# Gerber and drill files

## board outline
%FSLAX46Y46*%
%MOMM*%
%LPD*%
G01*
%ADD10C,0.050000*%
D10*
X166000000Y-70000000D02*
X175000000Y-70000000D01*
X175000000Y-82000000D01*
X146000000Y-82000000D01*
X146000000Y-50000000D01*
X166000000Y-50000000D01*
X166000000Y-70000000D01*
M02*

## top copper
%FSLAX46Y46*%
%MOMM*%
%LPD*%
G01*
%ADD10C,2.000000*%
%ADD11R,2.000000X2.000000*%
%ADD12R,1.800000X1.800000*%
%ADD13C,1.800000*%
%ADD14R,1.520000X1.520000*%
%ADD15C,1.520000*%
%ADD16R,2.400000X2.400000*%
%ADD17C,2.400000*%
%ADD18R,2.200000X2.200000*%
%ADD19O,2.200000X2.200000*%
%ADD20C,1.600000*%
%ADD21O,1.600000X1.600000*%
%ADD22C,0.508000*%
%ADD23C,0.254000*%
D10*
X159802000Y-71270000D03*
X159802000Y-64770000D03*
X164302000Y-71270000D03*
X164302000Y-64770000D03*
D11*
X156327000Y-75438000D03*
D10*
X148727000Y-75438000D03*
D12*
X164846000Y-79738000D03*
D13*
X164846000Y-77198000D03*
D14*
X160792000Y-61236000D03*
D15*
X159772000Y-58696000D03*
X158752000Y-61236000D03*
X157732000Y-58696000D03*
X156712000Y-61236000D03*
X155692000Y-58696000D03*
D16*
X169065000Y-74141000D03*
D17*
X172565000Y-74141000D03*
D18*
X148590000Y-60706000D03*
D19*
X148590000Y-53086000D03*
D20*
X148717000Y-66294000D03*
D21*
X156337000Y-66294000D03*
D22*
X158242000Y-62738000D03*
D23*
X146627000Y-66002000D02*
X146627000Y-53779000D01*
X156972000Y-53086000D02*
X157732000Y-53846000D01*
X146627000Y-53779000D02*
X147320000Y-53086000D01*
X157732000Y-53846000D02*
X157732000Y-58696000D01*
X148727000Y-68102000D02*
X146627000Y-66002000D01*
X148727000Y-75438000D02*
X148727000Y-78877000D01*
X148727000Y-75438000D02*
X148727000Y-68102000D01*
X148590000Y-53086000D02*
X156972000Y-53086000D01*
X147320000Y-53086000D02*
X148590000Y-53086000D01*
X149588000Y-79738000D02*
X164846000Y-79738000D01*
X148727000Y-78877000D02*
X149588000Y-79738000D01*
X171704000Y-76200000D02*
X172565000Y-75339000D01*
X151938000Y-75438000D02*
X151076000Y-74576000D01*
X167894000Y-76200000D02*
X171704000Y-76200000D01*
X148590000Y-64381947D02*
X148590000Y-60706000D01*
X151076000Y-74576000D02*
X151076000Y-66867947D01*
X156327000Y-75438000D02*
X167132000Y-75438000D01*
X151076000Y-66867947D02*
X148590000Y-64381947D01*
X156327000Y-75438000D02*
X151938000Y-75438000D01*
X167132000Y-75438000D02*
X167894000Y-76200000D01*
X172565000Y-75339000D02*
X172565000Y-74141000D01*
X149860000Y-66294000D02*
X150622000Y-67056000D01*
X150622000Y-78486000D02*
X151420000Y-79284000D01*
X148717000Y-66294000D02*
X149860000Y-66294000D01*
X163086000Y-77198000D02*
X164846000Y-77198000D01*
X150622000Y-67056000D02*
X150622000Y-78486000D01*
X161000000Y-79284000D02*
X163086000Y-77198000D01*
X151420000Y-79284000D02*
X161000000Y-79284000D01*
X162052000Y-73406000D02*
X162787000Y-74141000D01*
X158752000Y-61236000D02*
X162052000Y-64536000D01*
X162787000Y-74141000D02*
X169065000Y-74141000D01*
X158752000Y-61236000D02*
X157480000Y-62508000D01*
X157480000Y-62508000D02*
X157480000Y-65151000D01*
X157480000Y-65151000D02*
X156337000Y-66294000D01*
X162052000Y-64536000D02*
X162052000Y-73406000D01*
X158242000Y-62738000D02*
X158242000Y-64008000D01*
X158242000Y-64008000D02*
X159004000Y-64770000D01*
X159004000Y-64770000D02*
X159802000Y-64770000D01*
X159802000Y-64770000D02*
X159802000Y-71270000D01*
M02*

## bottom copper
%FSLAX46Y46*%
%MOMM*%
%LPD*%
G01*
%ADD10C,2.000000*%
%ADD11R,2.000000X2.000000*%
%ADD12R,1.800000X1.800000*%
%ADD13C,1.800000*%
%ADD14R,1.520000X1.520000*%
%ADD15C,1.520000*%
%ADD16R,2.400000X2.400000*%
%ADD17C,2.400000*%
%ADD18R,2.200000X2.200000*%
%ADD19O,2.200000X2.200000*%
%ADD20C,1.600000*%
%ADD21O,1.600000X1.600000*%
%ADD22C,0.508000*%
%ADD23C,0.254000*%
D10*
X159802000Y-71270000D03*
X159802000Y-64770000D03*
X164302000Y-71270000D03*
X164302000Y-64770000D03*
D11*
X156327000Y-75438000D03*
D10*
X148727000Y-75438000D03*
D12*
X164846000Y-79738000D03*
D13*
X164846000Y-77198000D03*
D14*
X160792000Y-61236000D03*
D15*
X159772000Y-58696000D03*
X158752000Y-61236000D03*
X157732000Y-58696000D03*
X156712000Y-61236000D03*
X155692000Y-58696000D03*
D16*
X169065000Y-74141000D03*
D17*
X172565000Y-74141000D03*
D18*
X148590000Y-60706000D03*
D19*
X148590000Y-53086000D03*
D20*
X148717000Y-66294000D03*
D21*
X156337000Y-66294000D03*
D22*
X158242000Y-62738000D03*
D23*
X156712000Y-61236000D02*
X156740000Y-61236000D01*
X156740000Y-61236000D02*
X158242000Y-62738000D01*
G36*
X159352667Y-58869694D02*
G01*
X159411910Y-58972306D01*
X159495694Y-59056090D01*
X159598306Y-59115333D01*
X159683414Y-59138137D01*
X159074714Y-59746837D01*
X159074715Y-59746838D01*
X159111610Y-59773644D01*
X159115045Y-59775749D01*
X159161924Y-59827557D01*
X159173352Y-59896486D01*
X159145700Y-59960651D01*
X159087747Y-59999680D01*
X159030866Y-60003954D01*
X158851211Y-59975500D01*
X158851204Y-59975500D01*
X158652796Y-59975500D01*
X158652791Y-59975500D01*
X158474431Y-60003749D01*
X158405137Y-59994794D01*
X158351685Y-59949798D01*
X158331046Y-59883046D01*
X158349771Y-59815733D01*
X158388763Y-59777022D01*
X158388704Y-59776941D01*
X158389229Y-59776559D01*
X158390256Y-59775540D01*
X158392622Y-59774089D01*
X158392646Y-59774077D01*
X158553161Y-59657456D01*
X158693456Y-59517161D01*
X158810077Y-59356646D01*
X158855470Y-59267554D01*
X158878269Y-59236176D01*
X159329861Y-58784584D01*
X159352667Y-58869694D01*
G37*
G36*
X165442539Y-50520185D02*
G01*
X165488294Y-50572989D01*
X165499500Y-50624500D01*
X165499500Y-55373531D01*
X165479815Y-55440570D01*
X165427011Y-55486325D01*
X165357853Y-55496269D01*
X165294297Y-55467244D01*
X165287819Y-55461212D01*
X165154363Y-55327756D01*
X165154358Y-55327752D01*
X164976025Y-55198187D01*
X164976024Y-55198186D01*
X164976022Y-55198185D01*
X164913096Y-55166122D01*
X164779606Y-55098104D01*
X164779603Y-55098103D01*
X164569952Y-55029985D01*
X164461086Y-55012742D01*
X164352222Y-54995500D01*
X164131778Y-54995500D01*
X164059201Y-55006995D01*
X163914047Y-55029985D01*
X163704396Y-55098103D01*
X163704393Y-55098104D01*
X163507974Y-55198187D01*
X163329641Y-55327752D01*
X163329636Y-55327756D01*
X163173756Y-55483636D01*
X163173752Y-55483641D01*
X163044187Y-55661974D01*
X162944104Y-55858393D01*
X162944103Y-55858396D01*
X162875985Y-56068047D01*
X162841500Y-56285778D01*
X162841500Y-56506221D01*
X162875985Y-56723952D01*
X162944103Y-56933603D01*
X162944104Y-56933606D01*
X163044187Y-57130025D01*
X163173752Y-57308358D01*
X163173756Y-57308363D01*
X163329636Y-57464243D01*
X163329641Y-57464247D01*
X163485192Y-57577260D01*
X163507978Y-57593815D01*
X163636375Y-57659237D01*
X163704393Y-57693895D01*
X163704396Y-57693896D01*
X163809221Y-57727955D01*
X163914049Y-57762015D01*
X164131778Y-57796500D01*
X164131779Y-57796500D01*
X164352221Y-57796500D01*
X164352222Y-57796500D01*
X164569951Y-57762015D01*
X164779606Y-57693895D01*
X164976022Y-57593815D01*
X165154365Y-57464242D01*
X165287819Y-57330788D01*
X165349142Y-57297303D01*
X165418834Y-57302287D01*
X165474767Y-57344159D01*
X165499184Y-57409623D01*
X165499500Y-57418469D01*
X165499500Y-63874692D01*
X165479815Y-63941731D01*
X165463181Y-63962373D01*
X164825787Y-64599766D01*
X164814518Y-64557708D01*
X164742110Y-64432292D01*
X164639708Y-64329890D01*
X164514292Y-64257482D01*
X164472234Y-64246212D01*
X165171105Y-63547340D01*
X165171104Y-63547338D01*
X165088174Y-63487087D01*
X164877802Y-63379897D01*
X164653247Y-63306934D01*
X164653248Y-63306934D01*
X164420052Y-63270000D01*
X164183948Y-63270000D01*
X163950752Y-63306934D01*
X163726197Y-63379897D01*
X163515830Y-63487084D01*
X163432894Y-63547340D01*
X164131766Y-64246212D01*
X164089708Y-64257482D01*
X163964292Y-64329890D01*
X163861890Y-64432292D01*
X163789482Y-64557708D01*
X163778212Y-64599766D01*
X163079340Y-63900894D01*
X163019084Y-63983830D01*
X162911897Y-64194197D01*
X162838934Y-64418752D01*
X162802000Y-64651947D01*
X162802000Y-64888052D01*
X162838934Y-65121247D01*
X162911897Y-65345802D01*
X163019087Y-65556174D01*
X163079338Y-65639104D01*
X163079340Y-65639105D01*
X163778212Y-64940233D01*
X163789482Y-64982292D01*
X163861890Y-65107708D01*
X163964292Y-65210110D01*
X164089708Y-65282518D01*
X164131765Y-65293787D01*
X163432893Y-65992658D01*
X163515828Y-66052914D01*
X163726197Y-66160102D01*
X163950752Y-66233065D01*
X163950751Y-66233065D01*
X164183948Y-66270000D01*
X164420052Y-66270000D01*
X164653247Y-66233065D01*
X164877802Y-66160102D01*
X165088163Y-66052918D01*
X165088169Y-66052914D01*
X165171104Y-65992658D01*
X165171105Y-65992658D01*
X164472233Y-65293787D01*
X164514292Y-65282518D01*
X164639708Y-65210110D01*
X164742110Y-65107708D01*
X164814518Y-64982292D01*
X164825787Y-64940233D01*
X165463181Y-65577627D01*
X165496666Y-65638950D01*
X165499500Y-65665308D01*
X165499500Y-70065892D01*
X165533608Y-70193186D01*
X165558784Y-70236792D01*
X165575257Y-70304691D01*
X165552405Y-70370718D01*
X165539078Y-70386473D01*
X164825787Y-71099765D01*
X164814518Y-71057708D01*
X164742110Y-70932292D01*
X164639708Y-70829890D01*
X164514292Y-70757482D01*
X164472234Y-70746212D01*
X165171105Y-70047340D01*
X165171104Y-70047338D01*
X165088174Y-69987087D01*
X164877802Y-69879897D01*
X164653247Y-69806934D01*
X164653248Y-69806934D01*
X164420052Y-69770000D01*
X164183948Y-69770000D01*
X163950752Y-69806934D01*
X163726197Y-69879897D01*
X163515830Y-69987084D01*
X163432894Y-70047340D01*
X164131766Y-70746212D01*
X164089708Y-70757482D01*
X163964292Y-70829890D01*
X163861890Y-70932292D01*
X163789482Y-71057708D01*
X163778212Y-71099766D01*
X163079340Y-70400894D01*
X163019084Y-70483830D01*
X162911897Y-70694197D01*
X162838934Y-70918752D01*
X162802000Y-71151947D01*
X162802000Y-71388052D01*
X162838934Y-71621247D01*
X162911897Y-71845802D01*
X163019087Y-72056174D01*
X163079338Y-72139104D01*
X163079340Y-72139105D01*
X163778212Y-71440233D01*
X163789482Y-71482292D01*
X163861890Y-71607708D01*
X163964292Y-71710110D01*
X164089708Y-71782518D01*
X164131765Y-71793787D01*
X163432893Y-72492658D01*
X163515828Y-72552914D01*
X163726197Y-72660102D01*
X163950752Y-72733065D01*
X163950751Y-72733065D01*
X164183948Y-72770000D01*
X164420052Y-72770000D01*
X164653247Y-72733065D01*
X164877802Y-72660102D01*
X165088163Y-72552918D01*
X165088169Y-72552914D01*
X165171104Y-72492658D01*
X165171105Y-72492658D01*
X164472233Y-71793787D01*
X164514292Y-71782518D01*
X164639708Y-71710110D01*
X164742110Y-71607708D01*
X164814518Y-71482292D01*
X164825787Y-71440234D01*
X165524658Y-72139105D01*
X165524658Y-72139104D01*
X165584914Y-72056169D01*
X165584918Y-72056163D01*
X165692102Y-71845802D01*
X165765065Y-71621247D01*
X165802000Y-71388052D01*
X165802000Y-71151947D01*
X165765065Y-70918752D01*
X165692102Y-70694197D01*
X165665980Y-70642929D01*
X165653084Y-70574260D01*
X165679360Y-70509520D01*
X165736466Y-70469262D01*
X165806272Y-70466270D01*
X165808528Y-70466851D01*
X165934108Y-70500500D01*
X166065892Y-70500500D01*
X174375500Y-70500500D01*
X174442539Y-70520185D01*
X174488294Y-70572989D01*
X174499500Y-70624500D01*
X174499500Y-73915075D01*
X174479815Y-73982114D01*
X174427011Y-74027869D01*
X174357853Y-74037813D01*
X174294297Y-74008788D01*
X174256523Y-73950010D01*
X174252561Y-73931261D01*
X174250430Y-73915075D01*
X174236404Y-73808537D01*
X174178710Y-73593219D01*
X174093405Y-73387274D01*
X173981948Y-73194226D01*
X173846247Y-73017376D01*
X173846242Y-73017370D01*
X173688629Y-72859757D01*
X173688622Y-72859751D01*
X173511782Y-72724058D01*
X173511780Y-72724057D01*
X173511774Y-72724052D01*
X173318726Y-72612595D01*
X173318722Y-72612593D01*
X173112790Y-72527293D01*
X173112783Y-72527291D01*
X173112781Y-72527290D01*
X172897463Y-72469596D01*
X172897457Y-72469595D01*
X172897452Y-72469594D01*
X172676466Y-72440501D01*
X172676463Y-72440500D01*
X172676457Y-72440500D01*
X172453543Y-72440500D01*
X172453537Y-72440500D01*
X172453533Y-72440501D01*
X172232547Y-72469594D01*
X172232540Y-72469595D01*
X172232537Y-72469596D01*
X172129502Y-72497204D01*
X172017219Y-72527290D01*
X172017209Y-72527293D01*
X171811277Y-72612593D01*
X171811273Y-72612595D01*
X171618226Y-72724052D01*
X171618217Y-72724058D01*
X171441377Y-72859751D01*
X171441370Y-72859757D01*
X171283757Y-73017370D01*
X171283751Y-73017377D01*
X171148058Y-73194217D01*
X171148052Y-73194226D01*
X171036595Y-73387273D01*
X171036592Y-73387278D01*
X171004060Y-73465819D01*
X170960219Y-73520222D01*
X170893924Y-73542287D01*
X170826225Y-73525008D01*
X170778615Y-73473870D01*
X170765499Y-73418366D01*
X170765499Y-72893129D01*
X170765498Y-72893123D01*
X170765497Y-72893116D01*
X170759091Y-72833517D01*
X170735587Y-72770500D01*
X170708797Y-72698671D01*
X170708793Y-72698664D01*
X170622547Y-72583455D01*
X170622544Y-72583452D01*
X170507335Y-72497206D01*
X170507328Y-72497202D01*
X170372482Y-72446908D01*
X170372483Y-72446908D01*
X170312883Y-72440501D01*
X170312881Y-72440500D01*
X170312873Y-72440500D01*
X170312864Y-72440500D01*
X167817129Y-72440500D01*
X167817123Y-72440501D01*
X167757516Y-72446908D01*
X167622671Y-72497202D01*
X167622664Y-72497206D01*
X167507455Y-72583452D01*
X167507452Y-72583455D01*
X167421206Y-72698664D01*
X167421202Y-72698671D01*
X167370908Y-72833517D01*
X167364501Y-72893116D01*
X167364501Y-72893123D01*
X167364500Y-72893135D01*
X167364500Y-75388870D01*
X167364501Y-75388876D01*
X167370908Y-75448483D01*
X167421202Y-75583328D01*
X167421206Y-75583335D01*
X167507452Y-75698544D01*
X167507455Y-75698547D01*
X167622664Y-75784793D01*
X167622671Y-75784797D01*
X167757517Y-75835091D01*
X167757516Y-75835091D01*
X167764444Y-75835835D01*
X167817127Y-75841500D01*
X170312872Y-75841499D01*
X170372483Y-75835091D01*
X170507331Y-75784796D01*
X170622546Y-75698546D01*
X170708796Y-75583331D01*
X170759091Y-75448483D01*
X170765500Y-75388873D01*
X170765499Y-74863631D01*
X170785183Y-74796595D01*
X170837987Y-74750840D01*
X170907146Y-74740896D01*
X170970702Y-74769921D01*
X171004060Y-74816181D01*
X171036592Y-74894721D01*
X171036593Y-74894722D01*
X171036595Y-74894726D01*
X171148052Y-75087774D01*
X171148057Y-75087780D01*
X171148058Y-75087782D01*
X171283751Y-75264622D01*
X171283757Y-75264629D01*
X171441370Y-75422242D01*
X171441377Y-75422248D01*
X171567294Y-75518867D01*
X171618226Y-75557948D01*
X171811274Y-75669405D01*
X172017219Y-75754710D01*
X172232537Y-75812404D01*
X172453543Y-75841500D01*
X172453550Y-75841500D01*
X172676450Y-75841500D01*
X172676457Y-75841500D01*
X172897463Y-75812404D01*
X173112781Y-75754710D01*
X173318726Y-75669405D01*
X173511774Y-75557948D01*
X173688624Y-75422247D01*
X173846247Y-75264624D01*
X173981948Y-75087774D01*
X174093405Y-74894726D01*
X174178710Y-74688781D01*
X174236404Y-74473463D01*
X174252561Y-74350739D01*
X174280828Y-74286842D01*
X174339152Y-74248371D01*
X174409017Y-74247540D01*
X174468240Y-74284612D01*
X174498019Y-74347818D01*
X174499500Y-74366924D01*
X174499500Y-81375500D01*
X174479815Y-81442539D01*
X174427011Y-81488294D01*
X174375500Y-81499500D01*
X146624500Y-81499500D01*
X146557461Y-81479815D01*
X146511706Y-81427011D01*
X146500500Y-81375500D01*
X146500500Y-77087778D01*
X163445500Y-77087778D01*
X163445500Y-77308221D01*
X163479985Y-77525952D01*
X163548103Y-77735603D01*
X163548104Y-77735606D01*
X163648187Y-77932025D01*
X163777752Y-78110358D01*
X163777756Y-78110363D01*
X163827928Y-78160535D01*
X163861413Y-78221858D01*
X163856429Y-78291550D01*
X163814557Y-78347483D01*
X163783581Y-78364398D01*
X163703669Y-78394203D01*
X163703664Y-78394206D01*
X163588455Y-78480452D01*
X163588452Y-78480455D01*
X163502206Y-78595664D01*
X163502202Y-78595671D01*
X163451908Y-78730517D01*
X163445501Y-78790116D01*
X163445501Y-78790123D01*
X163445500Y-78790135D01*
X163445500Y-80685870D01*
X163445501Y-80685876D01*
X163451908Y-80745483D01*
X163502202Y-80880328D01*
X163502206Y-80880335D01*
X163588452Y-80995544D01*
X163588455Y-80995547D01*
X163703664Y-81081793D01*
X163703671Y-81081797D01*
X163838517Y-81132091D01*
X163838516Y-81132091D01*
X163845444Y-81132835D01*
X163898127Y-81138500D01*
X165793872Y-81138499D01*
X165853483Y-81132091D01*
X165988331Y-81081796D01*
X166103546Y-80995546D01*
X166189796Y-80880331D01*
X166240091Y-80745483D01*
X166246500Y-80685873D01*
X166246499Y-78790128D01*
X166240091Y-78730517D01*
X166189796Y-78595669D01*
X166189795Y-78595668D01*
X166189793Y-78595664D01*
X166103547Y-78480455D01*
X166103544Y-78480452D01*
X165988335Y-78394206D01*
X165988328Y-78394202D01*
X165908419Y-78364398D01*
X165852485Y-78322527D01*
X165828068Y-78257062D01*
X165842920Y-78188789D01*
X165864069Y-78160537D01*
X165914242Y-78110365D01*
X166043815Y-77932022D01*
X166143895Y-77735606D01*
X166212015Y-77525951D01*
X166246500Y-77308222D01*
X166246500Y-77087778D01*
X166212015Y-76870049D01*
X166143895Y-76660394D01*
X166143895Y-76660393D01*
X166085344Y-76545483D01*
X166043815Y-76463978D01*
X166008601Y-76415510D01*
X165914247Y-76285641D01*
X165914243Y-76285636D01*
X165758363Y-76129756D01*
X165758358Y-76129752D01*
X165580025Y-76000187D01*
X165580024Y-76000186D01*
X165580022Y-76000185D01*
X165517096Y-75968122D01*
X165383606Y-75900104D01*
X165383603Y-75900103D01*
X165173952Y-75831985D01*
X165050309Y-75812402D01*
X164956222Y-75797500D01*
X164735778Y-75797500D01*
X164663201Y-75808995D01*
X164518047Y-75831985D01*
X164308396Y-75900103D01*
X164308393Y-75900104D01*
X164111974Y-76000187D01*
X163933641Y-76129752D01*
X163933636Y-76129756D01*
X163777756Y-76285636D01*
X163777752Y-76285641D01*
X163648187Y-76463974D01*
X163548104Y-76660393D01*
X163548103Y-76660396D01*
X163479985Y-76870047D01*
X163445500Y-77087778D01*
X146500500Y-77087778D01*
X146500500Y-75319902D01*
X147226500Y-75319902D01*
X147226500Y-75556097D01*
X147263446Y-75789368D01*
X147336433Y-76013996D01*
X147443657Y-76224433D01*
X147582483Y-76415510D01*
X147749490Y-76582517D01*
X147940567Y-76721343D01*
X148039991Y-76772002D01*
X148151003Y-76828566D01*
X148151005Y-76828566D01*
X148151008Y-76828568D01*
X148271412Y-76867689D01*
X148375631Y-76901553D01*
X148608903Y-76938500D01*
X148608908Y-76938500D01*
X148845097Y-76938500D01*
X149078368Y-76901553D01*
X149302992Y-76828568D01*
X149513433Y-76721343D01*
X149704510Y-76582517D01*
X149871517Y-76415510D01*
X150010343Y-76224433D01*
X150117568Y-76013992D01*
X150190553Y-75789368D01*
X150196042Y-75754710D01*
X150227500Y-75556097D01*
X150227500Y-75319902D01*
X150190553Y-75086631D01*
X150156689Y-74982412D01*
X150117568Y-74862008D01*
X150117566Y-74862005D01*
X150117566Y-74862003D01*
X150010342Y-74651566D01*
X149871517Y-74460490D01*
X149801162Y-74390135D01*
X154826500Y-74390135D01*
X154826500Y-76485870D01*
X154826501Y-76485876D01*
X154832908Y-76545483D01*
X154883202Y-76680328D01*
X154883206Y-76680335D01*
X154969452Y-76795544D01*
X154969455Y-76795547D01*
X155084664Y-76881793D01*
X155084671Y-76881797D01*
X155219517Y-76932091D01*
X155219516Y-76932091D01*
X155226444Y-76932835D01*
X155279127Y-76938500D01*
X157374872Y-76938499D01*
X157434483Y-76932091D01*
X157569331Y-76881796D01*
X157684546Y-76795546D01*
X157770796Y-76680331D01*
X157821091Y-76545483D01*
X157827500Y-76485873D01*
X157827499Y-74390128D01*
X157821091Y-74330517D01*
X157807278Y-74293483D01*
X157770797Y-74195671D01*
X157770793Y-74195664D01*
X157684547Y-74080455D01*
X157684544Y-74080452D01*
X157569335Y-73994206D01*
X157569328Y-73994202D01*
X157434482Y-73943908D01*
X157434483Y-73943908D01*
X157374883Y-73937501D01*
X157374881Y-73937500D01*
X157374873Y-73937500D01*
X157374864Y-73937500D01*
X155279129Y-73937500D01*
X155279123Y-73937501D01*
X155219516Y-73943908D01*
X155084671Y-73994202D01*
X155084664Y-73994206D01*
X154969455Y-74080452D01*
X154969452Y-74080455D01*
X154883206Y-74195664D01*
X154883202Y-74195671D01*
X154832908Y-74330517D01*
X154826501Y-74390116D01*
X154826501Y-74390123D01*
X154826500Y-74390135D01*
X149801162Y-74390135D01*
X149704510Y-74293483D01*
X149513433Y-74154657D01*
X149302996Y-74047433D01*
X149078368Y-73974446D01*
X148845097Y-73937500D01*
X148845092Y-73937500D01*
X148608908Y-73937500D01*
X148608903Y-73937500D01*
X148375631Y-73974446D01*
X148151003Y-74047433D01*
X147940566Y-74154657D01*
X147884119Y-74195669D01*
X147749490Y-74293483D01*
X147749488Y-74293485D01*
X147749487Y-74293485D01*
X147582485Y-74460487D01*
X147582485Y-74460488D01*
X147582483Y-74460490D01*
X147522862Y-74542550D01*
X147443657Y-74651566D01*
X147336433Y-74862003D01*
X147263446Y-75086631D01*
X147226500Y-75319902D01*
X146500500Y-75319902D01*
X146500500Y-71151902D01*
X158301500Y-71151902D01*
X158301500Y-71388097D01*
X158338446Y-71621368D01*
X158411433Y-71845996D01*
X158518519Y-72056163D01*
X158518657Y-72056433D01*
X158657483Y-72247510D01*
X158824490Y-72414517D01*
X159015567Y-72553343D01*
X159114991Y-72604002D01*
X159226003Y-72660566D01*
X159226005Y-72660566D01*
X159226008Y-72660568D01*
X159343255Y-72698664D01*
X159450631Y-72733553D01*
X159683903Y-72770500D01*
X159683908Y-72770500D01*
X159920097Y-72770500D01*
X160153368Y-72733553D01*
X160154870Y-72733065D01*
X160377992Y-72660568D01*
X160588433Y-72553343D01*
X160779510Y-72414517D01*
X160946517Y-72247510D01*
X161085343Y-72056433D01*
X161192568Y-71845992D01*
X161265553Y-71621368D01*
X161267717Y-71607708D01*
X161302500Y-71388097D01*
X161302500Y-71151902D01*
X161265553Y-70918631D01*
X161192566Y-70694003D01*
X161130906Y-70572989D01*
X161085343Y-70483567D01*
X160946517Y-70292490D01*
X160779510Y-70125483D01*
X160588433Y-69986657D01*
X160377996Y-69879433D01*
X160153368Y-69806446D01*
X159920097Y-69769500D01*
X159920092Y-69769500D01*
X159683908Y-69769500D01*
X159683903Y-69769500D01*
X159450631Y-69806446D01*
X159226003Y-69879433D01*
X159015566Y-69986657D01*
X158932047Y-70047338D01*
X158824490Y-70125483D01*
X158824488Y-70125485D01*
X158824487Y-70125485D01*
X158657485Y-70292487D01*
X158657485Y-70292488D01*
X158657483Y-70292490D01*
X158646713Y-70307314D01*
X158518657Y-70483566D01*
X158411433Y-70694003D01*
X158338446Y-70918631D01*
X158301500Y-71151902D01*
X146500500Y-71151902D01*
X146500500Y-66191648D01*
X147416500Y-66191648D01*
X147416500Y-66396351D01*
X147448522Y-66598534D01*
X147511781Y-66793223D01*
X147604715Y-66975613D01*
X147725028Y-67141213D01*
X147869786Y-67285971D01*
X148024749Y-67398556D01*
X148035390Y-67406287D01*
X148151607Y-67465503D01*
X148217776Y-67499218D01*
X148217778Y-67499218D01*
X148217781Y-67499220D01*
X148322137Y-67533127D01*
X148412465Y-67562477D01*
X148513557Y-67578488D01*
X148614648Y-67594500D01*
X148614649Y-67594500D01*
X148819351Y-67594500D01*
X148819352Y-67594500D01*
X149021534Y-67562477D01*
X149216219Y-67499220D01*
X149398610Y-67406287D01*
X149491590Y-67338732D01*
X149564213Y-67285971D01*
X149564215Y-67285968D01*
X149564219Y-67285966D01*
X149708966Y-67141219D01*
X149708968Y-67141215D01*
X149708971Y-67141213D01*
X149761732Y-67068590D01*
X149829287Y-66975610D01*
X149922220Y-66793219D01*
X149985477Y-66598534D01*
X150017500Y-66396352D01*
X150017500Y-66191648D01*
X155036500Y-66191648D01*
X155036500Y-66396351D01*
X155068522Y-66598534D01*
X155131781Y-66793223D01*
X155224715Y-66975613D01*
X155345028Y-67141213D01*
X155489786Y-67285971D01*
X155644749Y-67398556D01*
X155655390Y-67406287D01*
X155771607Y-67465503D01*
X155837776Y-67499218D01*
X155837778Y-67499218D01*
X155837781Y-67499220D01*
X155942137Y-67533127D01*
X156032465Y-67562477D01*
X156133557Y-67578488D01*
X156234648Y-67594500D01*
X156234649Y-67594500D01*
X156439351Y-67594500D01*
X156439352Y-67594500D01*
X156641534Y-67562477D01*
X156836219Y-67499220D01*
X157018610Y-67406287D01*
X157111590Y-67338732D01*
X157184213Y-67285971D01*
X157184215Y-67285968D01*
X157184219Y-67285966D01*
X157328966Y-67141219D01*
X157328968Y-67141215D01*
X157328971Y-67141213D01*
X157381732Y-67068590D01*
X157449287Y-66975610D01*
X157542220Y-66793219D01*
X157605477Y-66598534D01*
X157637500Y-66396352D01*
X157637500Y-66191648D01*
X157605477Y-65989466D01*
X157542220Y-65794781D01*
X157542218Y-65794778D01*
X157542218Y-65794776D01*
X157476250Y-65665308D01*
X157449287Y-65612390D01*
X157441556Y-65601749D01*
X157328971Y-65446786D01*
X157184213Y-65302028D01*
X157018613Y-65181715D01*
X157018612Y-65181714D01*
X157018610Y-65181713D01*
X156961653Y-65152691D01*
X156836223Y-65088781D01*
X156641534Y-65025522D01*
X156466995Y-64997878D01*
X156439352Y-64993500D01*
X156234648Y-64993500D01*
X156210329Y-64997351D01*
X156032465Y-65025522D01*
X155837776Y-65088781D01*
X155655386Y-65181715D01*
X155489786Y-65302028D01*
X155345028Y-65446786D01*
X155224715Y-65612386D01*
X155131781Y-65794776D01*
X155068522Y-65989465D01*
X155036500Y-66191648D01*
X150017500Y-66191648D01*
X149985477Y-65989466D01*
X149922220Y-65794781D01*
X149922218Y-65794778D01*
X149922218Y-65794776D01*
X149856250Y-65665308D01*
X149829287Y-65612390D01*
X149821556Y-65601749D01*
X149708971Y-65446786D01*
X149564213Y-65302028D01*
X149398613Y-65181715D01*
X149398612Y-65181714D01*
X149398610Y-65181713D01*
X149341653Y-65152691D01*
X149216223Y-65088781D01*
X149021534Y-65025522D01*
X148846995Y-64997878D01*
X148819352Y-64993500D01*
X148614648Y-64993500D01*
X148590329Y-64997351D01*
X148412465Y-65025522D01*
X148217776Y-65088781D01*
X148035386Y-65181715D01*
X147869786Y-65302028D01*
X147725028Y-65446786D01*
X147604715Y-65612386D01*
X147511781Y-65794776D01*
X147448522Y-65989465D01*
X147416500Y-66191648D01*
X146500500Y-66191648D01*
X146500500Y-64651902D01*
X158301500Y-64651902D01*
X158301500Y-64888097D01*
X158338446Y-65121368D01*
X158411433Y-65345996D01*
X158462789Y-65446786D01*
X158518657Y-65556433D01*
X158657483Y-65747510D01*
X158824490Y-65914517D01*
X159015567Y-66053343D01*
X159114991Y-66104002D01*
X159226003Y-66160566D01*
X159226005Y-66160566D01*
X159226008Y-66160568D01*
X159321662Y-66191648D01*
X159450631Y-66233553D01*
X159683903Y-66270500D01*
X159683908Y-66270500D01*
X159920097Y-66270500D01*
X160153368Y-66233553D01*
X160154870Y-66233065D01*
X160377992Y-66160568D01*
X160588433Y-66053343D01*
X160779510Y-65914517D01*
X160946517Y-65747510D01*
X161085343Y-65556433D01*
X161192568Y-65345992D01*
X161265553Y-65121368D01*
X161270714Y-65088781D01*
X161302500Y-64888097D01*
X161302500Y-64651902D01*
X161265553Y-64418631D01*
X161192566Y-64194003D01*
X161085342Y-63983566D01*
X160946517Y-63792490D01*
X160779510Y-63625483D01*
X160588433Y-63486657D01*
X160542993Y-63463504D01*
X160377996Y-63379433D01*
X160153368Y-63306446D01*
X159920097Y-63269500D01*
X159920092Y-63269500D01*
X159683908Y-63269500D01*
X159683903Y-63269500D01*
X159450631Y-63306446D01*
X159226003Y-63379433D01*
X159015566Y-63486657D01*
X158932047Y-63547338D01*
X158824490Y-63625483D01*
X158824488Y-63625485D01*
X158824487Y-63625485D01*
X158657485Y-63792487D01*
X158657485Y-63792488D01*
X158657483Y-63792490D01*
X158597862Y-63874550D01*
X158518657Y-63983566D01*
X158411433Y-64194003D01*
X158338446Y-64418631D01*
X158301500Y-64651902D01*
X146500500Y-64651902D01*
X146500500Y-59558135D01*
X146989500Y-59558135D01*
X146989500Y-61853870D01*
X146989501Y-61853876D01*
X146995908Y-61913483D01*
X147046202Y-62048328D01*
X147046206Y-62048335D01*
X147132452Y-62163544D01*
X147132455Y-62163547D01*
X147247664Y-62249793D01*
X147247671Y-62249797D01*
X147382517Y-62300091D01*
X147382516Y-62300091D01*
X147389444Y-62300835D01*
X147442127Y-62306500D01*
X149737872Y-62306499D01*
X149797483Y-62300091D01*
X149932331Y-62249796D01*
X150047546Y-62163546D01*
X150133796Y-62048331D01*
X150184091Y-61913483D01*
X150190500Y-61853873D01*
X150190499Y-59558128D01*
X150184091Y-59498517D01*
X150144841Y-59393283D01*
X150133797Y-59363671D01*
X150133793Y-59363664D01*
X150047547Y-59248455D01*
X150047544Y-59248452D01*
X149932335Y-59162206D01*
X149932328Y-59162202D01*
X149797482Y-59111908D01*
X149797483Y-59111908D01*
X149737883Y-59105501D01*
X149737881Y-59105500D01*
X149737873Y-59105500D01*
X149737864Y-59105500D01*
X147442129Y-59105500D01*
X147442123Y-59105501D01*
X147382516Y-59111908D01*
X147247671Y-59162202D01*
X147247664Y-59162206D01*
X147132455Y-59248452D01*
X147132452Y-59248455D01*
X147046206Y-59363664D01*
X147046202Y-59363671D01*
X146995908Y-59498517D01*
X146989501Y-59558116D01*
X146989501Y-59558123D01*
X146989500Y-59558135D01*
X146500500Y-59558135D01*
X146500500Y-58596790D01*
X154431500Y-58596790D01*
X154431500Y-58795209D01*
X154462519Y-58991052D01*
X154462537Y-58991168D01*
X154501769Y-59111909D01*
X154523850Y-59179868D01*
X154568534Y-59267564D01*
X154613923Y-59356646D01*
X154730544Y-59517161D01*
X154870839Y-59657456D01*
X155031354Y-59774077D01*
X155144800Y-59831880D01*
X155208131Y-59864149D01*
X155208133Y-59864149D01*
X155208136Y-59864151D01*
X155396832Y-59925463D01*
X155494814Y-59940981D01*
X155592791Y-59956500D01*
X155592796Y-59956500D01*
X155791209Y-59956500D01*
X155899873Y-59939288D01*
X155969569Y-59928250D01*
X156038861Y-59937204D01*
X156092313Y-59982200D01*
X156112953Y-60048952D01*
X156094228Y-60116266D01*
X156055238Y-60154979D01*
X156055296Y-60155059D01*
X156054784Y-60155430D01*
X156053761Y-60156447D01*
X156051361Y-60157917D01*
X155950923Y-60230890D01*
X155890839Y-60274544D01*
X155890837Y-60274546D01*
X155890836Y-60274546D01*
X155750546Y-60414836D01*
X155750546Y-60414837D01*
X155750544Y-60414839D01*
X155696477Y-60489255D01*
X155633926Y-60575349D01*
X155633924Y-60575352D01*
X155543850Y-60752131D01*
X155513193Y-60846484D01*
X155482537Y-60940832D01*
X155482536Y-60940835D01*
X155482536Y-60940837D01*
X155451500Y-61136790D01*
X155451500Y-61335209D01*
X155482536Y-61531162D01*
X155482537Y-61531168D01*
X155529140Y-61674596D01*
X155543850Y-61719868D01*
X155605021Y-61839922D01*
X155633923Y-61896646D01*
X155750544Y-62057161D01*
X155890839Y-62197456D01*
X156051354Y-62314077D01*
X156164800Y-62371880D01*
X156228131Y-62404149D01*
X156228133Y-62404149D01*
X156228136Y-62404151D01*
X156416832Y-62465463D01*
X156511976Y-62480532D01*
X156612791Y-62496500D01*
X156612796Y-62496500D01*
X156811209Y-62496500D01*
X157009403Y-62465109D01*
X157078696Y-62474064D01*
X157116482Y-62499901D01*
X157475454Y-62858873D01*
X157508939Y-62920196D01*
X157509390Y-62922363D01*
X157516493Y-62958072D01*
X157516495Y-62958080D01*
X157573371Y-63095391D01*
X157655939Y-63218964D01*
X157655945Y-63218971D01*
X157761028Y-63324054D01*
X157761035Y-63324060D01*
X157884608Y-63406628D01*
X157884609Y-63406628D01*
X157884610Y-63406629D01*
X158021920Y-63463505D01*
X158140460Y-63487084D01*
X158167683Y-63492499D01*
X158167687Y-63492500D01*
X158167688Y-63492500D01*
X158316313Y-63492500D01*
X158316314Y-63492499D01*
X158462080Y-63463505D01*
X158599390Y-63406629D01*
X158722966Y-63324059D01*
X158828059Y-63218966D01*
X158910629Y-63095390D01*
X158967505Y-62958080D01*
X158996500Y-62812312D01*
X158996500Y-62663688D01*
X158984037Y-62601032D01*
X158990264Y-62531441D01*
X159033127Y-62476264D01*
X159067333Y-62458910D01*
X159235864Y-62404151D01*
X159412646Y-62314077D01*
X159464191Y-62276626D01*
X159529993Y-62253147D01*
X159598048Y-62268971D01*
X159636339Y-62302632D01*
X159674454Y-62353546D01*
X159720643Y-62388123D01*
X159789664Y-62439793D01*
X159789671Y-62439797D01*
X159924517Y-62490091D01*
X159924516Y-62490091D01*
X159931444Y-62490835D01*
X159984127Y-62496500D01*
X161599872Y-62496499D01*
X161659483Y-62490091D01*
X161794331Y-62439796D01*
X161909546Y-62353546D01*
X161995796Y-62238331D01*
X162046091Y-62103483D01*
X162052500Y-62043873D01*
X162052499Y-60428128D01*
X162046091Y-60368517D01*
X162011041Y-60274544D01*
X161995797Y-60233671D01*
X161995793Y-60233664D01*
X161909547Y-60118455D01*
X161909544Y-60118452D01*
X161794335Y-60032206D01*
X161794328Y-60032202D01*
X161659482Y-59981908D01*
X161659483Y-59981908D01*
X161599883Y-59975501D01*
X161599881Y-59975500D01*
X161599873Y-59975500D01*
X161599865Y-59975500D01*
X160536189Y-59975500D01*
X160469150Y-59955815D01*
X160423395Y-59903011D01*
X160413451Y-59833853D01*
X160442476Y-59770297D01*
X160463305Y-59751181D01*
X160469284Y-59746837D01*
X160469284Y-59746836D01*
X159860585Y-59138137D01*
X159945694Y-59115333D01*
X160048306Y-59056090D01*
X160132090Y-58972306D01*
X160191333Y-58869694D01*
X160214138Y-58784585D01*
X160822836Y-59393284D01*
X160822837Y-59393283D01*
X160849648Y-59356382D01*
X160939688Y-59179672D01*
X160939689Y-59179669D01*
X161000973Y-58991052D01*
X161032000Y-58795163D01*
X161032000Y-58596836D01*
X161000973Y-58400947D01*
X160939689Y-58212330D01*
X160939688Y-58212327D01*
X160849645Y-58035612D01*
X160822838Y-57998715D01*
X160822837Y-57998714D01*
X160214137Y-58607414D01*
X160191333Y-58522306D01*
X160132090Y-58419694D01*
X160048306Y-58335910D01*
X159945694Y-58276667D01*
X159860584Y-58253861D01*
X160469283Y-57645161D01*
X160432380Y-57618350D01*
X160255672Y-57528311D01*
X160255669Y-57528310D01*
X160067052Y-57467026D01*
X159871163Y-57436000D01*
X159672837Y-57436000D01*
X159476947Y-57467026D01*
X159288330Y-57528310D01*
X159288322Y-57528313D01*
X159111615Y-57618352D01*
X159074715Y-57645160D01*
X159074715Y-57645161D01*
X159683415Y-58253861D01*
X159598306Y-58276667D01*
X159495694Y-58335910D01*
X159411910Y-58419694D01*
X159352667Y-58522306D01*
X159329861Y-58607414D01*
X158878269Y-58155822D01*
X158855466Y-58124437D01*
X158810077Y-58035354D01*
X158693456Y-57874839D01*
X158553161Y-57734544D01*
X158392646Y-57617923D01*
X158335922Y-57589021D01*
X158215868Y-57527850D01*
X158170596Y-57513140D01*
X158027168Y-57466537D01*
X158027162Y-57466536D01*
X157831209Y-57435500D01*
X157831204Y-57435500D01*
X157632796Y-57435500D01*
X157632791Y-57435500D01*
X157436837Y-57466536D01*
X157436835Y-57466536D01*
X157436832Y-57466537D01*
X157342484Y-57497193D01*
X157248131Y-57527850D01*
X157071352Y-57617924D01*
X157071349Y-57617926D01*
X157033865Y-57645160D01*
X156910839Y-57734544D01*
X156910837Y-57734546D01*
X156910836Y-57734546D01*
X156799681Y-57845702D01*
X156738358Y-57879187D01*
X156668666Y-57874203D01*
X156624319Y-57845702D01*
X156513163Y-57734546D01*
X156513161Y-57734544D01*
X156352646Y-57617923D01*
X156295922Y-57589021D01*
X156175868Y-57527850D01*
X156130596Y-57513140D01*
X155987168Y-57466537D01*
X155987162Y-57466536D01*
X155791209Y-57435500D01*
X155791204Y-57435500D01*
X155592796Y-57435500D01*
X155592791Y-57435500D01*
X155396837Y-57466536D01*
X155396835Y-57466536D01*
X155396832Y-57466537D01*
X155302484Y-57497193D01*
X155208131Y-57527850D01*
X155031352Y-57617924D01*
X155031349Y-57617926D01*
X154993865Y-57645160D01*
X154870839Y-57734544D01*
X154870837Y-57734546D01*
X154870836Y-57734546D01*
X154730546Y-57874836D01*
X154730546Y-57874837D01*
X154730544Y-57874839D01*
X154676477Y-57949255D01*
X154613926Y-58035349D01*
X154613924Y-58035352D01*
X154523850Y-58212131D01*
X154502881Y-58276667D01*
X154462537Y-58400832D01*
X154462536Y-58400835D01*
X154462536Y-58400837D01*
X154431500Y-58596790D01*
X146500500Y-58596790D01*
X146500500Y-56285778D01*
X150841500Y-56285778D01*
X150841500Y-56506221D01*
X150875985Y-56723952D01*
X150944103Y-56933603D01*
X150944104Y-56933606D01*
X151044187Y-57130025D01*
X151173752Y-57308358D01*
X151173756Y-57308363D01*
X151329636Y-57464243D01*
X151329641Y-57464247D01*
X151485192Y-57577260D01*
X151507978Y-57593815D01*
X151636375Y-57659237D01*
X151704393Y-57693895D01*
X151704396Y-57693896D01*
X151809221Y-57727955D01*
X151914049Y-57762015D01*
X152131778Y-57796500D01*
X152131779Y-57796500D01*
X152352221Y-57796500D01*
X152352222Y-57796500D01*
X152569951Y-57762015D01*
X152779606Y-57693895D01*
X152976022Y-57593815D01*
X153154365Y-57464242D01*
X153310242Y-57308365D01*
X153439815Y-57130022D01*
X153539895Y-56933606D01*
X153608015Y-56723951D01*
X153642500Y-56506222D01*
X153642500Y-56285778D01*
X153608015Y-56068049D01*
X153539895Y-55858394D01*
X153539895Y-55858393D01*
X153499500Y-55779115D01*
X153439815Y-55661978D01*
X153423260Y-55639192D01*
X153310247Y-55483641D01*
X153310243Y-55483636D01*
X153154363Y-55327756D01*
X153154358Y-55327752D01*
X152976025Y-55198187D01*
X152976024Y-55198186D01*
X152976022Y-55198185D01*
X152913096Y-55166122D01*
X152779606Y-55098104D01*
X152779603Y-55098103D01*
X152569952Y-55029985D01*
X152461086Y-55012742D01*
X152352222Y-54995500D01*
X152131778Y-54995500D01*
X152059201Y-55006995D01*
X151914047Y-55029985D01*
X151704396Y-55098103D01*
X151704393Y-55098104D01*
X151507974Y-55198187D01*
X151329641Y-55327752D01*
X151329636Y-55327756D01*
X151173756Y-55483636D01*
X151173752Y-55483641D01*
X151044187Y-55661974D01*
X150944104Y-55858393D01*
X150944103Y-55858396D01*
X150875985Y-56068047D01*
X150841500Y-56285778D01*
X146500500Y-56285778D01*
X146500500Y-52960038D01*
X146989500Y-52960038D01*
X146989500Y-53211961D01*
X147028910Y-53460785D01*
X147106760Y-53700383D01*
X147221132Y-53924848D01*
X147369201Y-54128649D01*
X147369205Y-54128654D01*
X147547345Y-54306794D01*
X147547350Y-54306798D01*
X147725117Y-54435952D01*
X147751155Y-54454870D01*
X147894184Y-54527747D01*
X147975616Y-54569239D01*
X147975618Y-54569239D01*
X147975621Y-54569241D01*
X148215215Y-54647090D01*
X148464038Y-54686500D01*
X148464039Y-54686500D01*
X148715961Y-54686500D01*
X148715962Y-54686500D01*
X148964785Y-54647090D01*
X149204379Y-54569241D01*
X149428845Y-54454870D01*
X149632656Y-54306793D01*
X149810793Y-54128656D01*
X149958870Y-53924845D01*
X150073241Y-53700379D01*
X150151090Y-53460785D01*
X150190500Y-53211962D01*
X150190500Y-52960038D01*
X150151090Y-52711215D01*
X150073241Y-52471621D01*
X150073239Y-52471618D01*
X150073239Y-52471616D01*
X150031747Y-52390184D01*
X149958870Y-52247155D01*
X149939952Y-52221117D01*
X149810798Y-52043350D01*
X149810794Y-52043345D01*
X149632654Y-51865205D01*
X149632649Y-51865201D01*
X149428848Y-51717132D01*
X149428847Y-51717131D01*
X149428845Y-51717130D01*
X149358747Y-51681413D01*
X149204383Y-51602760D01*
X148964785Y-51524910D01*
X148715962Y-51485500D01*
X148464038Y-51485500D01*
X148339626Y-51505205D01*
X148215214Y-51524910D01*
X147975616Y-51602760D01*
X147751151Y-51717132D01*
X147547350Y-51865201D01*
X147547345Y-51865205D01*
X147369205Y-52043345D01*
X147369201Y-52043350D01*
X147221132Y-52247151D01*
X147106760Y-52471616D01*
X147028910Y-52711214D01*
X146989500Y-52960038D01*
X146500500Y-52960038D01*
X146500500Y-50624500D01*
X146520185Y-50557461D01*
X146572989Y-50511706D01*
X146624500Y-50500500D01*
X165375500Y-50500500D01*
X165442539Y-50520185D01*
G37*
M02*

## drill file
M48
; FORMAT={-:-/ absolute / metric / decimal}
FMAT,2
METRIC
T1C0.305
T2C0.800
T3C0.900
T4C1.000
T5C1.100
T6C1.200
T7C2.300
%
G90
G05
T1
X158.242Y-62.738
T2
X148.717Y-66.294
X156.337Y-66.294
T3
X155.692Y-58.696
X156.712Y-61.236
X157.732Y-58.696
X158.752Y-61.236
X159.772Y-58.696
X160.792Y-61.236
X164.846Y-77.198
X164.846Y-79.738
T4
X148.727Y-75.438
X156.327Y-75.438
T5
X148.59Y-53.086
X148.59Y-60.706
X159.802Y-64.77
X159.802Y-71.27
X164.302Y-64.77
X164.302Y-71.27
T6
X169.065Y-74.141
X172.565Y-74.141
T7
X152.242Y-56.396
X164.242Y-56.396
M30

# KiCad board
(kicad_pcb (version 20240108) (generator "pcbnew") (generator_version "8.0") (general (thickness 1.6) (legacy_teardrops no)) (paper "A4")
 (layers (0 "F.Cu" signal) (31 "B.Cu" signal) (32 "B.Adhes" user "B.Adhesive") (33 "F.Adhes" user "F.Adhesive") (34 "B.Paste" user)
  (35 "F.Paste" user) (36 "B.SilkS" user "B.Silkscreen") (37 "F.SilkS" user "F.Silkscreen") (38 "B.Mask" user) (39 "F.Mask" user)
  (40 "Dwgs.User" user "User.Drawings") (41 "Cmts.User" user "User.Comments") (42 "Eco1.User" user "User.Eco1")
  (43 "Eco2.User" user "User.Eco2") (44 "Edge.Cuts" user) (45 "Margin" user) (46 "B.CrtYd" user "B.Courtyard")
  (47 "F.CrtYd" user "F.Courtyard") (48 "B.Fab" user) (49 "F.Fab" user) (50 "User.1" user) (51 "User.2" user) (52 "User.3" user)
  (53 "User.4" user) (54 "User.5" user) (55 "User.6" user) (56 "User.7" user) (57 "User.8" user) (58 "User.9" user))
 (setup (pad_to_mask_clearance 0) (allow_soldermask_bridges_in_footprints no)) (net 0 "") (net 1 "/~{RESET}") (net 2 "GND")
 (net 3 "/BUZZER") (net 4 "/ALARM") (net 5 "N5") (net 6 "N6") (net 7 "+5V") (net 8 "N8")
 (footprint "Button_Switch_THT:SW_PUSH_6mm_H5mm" (layer "F.Cu") (at 159.802 71.27 90)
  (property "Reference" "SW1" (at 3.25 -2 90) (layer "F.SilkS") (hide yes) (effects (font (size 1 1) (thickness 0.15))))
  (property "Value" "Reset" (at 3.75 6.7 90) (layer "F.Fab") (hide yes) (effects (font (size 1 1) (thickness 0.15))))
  (pad "1" thru_hole circle (at 0 0 180) (size 2 2) (drill 1.1) (layers "*.Cu" "*.Mask") (remove_unused_layers no) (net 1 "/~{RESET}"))
  (pad "1" thru_hole circle (at 6.5 0 180) (size 2 2) (drill 1.1) (layers "*.Cu" "*.Mask") (remove_unused_layers no) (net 1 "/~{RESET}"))
  (pad "2" thru_hole circle (at 0 4.5 180) (size 2 2) (drill 1.1) (layers "*.Cu" "*.Mask") (remove_unused_layers no) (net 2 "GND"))
  (pad "2" thru_hole circle (at 6.5 4.5 180) (size 2 2) (drill 1.1) (layers "*.Cu" "*.Mask") (remove_unused_layers no) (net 2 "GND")))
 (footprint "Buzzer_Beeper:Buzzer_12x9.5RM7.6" (layer "F.Cu") (at 156.327 75.438 180)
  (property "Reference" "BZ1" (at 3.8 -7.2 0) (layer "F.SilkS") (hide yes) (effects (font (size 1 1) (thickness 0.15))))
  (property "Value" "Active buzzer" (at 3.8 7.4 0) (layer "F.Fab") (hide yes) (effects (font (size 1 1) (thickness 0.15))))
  (pad "1" thru_hole rect (at 0 0 180) (size 2 2) (drill 1) (layers "*.Cu" "*.Mask") (remove_unused_layers no) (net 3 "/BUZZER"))
  (pad "2" thru_hole circle (at 7.6 0 180) (size 2 2) (drill 1) (layers "*.Cu" "*.Mask") (remove_unused_layers no) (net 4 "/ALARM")))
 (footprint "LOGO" (layer "F.Cu") (at 158 54.25)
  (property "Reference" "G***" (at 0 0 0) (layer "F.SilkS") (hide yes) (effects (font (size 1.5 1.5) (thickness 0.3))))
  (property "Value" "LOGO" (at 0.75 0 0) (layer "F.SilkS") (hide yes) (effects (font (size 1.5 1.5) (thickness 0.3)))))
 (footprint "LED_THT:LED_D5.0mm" (layer "F.Cu") (at 164.846 79.738 90)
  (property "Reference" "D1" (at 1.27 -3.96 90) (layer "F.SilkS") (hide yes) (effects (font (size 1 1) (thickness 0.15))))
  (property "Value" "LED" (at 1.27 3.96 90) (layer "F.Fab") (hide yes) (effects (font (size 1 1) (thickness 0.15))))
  (pad "1" thru_hole rect (at 0 0 90) (size 1.8 1.8) (drill 0.9) (layers "*.Cu" "*.Mask") (remove_unused_layers no) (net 4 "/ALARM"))
  (pad "2" thru_hole circle (at 2.54 0 90) (size 1.8 1.8) (drill 0.9) (layers "*.Cu" "*.Mask") (remove_unused_layers no) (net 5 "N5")))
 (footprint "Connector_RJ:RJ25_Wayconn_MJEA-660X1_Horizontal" (layer "B.Cu") (at 160.792 61.236)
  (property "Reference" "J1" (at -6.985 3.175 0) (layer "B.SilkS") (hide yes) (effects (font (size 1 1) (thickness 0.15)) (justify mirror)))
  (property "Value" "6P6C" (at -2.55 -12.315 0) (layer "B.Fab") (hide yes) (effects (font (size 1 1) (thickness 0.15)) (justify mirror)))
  (pad "" np_thru_hole circle (at -8.55 -4.84) (size 2.3 2.3) (drill 2.3) (layers "*.Cu" "*.Mask"))
  (pad "" np_thru_hole circle (at 3.45 -4.84) (size 2.3 2.3) (drill 2.3) (layers "*.Cu" "*.Mask"))
  (pad "1" thru_hole rect (at 0 0) (size 1.52 1.52) (drill 0.9) (layers "*.Cu" "*.Mask") (remove_unused_layers no) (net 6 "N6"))
  (pad "2" thru_hole circle (at -1.02 -2.54) (size 1.52 1.52) (drill 0.9) (layers "*.Cu" "*.Mask") (remove_unused_layers no) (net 2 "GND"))
  (pad "3" thru_hole circle (at -2.04 0) (size 1.52 1.52) (drill 0.9) (layers "*.Cu" "*.Mask") (remove_unused_layers no) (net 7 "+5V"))
  (pad "4" thru_hole circle (at -3.06 -2.54) (size 1.52 1.52) (drill 0.9) (layers "*.Cu" "*.Mask") (remove_unused_layers no)
   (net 4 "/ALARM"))
  (pad "5" thru_hole circle (at -4.08 0) (size 1.52 1.52) (drill 0.9) (layers "*.Cu" "*.Mask") (remove_unused_layers no) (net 1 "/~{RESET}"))
  (pad "6" thru_hole circle (at -5.1 -2.54) (size 1.52 1.52) (drill 0.9) (layers "*.Cu" "*.Mask") (remove_unused_layers no) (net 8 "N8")))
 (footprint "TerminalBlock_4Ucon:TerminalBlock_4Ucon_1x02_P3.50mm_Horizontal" (layer "B.Cu") (at 169.065 74.141)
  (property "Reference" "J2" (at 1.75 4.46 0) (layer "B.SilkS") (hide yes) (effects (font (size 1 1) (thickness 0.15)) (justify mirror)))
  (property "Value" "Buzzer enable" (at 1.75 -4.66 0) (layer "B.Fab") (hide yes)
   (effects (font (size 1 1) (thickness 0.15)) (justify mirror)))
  (pad "1" thru_hole rect (at 0 0) (size 2.4 2.4) (drill 1.2) (layers "*.Cu" "*.Mask") (remove_unused_layers no) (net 7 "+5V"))
  (pad "2" thru_hole circle (at 3.5 0) (size 2.4 2.4) (drill 1.2) (layers "*.Cu" "*.Mask") (remove_unused_layers no) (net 3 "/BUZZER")))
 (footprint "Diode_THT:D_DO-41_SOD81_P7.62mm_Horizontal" (layer "B.Cu") (at 148.59 60.706 90)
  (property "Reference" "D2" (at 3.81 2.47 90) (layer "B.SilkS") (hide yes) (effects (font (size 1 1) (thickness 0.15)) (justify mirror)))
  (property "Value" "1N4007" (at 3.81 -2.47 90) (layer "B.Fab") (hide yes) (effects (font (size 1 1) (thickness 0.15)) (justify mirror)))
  (pad "1" thru_hole rect (at 0 0 90) (size 2.2 2.2) (drill 1.1) (layers "*.Cu" "*.Mask") (remove_unused_layers no) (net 3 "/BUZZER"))
  (pad "2" thru_hole oval (at 7.62 0 90) (size 2.2 2.2) (drill 1.1) (layers "*.Cu" "*.Mask") (remove_unused_layers no) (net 4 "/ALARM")))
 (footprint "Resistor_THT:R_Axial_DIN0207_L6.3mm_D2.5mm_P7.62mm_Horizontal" (layer "B.Cu") (at 148.717 66.294)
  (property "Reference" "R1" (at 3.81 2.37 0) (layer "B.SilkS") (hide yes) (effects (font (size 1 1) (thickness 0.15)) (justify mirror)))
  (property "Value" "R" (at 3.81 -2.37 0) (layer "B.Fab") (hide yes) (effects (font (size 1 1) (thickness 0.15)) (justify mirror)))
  (pad "1" thru_hole circle (at 0 0) (size 1.6 1.6) (drill 0.8) (layers "*.Cu" "*.Mask") (remove_unused_layers no) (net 5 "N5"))
  (pad "2" thru_hole oval (at 7.62 0) (size 1.6 1.6) (drill 0.8) (layers "*.Cu" "*.Mask") (remove_unused_layers no) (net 7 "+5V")))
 (gr_poly
  (pts (xy 166 70) (xy 175 70) (xy 175 82) (xy 146 82) (xy 146 50) (xy 166 50)) (stroke (width 0.05) (type solid)) (fill none)
  (layer "Edge.Cuts"))
 (segment (start 146.627 66.002) (end 146.627 53.779) (width 0.254) (layer "F.Cu") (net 4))
 (segment (start 156.972 53.086) (end 157.732 53.846) (width 0.254) (layer "F.Cu") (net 4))
 (segment (start 146.627 53.779) (end 147.32 53.086) (width 0.254) (layer "F.Cu") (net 4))
 (segment (start 157.732 53.846) (end 157.732 58.696) (width 0.254) (layer "F.Cu") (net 4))
 (segment (start 148.727 68.102) (end 146.627 66.002) (width 0.254) (layer "F.Cu") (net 4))
 (segment (start 148.727 75.438) (end 148.727 78.877) (width 0.254) (layer "F.Cu") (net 4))
 (segment (start 148.727 75.438) (end 148.727 68.102) (width 0.254) (layer "F.Cu") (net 4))
 (segment (start 148.59 53.086) (end 156.972 53.086) (width 0.254) (layer "F.Cu") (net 4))
 (segment (start 147.32 53.086) (end 148.59 53.086) (width 0.254) (layer "F.Cu") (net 4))
 (segment (start 149.588 79.738) (end 164.846 79.738) (width 0.254) (layer "F.Cu") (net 4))
 (segment (start 148.727 78.877) (end 149.588 79.738) (width 0.254) (layer "F.Cu") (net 4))
 (segment (start 171.704 76.2) (end 172.565 75.339) (width 0.254) (layer "F.Cu") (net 3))
 (segment (start 151.938 75.438) (end 151.076 74.576) (width 0.254) (layer "F.Cu") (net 3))
 (segment (start 167.894 76.2) (end 171.704 76.2) (width 0.254) (layer "F.Cu") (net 3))
 (segment (start 148.59 64.381947) (end 148.59 60.706) (width 0.254) (layer "F.Cu") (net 3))
 (segment (start 151.076 74.576) (end 151.076 66.867947) (width 0.254) (layer "F.Cu") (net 3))
 (segment (start 156.327 75.438) (end 167.132 75.438) (width 0.254) (layer "F.Cu") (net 3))
 (segment (start 151.076 66.867947) (end 148.59 64.381947) (width 0.254) (layer "F.Cu") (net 3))
 (segment (start 156.327 75.438) (end 151.938 75.438) (width 0.254) (layer "F.Cu") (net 3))
 (segment (start 167.132 75.438) (end 167.894 76.2) (width 0.254) (layer "F.Cu") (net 3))
 (segment (start 172.565 75.339) (end 172.565 74.141) (width 0.254) (layer "F.Cu") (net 3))
 (segment (start 149.86 66.294) (end 150.622 67.056) (width 0.254) (layer "F.Cu") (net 5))
 (segment (start 150.622 78.486) (end 151.42 79.284) (width 0.254) (layer "F.Cu") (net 5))
 (segment (start 148.717 66.294) (end 149.86 66.294) (width 0.254) (layer "F.Cu") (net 5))
 (segment (start 163.086 77.198) (end 164.846 77.198) (width 0.254) (layer "F.Cu") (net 5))
 (segment (start 150.622 67.056) (end 150.622 78.486) (width 0.254) (layer "F.Cu") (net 5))
 (segment (start 161 79.284) (end 163.086 77.198) (width 0.254) (layer "F.Cu") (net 5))
 (segment (start 151.42 79.284) (end 161 79.284) (width 0.254) (layer "F.Cu") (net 5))
 (segment (start 162.052 73.406) (end 162.787 74.141) (width 0.254) (layer "F.Cu") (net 7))
 (segment (start 158.752 61.236) (end 162.052 64.536) (width 0.254) (layer "F.Cu") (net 7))
 (segment (start 162.787 74.141) (end 169.065 74.141) (width 0.254) (layer "F.Cu") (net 7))
 (segment (start 158.752 61.236) (end 157.48 62.508) (width 0.254) (layer "F.Cu") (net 7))
 (segment (start 157.48 62.508) (end 157.48 65.151) (width 0.254) (layer "F.Cu") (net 7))
 (segment (start 157.48 65.151) (end 156.337 66.294) (width 0.254) (layer "F.Cu") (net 7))
 (segment (start 162.052 64.536) (end 162.052 73.406) (width 0.254) (layer "F.Cu") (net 7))
 (segment (start 158.242 62.738) (end 158.242 64.008) (width 0.254) (layer "F.Cu") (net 1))
 (segment (start 158.242 64.008) (end 159.004 64.77) (width 0.254) (layer "F.Cu") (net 1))
 (segment (start 159.004 64.77) (end 159.802 64.77) (width 0.254) (layer "F.Cu") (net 1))
 (segment (start 159.802 64.77) (end 159.802 71.27) (width 0.254) (layer "F.Cu") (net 1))
 (via (at 158.242 62.738) (size 0.508) (drill 0.3048) (layers "F.Cu" "B.Cu") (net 1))
 (segment (start 156.712 61.236) (end 156.74 61.236) (width 0.254) (layer "B.Cu") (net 1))
 (segment (start 156.74 61.236) (end 158.242 62.738) (width 0.254) (layer "B.Cu") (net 1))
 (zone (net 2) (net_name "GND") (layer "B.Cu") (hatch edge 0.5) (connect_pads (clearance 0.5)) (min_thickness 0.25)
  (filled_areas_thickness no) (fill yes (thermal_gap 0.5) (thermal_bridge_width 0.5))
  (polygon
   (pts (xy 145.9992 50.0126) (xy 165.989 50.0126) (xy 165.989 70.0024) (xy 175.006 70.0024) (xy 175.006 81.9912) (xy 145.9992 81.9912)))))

